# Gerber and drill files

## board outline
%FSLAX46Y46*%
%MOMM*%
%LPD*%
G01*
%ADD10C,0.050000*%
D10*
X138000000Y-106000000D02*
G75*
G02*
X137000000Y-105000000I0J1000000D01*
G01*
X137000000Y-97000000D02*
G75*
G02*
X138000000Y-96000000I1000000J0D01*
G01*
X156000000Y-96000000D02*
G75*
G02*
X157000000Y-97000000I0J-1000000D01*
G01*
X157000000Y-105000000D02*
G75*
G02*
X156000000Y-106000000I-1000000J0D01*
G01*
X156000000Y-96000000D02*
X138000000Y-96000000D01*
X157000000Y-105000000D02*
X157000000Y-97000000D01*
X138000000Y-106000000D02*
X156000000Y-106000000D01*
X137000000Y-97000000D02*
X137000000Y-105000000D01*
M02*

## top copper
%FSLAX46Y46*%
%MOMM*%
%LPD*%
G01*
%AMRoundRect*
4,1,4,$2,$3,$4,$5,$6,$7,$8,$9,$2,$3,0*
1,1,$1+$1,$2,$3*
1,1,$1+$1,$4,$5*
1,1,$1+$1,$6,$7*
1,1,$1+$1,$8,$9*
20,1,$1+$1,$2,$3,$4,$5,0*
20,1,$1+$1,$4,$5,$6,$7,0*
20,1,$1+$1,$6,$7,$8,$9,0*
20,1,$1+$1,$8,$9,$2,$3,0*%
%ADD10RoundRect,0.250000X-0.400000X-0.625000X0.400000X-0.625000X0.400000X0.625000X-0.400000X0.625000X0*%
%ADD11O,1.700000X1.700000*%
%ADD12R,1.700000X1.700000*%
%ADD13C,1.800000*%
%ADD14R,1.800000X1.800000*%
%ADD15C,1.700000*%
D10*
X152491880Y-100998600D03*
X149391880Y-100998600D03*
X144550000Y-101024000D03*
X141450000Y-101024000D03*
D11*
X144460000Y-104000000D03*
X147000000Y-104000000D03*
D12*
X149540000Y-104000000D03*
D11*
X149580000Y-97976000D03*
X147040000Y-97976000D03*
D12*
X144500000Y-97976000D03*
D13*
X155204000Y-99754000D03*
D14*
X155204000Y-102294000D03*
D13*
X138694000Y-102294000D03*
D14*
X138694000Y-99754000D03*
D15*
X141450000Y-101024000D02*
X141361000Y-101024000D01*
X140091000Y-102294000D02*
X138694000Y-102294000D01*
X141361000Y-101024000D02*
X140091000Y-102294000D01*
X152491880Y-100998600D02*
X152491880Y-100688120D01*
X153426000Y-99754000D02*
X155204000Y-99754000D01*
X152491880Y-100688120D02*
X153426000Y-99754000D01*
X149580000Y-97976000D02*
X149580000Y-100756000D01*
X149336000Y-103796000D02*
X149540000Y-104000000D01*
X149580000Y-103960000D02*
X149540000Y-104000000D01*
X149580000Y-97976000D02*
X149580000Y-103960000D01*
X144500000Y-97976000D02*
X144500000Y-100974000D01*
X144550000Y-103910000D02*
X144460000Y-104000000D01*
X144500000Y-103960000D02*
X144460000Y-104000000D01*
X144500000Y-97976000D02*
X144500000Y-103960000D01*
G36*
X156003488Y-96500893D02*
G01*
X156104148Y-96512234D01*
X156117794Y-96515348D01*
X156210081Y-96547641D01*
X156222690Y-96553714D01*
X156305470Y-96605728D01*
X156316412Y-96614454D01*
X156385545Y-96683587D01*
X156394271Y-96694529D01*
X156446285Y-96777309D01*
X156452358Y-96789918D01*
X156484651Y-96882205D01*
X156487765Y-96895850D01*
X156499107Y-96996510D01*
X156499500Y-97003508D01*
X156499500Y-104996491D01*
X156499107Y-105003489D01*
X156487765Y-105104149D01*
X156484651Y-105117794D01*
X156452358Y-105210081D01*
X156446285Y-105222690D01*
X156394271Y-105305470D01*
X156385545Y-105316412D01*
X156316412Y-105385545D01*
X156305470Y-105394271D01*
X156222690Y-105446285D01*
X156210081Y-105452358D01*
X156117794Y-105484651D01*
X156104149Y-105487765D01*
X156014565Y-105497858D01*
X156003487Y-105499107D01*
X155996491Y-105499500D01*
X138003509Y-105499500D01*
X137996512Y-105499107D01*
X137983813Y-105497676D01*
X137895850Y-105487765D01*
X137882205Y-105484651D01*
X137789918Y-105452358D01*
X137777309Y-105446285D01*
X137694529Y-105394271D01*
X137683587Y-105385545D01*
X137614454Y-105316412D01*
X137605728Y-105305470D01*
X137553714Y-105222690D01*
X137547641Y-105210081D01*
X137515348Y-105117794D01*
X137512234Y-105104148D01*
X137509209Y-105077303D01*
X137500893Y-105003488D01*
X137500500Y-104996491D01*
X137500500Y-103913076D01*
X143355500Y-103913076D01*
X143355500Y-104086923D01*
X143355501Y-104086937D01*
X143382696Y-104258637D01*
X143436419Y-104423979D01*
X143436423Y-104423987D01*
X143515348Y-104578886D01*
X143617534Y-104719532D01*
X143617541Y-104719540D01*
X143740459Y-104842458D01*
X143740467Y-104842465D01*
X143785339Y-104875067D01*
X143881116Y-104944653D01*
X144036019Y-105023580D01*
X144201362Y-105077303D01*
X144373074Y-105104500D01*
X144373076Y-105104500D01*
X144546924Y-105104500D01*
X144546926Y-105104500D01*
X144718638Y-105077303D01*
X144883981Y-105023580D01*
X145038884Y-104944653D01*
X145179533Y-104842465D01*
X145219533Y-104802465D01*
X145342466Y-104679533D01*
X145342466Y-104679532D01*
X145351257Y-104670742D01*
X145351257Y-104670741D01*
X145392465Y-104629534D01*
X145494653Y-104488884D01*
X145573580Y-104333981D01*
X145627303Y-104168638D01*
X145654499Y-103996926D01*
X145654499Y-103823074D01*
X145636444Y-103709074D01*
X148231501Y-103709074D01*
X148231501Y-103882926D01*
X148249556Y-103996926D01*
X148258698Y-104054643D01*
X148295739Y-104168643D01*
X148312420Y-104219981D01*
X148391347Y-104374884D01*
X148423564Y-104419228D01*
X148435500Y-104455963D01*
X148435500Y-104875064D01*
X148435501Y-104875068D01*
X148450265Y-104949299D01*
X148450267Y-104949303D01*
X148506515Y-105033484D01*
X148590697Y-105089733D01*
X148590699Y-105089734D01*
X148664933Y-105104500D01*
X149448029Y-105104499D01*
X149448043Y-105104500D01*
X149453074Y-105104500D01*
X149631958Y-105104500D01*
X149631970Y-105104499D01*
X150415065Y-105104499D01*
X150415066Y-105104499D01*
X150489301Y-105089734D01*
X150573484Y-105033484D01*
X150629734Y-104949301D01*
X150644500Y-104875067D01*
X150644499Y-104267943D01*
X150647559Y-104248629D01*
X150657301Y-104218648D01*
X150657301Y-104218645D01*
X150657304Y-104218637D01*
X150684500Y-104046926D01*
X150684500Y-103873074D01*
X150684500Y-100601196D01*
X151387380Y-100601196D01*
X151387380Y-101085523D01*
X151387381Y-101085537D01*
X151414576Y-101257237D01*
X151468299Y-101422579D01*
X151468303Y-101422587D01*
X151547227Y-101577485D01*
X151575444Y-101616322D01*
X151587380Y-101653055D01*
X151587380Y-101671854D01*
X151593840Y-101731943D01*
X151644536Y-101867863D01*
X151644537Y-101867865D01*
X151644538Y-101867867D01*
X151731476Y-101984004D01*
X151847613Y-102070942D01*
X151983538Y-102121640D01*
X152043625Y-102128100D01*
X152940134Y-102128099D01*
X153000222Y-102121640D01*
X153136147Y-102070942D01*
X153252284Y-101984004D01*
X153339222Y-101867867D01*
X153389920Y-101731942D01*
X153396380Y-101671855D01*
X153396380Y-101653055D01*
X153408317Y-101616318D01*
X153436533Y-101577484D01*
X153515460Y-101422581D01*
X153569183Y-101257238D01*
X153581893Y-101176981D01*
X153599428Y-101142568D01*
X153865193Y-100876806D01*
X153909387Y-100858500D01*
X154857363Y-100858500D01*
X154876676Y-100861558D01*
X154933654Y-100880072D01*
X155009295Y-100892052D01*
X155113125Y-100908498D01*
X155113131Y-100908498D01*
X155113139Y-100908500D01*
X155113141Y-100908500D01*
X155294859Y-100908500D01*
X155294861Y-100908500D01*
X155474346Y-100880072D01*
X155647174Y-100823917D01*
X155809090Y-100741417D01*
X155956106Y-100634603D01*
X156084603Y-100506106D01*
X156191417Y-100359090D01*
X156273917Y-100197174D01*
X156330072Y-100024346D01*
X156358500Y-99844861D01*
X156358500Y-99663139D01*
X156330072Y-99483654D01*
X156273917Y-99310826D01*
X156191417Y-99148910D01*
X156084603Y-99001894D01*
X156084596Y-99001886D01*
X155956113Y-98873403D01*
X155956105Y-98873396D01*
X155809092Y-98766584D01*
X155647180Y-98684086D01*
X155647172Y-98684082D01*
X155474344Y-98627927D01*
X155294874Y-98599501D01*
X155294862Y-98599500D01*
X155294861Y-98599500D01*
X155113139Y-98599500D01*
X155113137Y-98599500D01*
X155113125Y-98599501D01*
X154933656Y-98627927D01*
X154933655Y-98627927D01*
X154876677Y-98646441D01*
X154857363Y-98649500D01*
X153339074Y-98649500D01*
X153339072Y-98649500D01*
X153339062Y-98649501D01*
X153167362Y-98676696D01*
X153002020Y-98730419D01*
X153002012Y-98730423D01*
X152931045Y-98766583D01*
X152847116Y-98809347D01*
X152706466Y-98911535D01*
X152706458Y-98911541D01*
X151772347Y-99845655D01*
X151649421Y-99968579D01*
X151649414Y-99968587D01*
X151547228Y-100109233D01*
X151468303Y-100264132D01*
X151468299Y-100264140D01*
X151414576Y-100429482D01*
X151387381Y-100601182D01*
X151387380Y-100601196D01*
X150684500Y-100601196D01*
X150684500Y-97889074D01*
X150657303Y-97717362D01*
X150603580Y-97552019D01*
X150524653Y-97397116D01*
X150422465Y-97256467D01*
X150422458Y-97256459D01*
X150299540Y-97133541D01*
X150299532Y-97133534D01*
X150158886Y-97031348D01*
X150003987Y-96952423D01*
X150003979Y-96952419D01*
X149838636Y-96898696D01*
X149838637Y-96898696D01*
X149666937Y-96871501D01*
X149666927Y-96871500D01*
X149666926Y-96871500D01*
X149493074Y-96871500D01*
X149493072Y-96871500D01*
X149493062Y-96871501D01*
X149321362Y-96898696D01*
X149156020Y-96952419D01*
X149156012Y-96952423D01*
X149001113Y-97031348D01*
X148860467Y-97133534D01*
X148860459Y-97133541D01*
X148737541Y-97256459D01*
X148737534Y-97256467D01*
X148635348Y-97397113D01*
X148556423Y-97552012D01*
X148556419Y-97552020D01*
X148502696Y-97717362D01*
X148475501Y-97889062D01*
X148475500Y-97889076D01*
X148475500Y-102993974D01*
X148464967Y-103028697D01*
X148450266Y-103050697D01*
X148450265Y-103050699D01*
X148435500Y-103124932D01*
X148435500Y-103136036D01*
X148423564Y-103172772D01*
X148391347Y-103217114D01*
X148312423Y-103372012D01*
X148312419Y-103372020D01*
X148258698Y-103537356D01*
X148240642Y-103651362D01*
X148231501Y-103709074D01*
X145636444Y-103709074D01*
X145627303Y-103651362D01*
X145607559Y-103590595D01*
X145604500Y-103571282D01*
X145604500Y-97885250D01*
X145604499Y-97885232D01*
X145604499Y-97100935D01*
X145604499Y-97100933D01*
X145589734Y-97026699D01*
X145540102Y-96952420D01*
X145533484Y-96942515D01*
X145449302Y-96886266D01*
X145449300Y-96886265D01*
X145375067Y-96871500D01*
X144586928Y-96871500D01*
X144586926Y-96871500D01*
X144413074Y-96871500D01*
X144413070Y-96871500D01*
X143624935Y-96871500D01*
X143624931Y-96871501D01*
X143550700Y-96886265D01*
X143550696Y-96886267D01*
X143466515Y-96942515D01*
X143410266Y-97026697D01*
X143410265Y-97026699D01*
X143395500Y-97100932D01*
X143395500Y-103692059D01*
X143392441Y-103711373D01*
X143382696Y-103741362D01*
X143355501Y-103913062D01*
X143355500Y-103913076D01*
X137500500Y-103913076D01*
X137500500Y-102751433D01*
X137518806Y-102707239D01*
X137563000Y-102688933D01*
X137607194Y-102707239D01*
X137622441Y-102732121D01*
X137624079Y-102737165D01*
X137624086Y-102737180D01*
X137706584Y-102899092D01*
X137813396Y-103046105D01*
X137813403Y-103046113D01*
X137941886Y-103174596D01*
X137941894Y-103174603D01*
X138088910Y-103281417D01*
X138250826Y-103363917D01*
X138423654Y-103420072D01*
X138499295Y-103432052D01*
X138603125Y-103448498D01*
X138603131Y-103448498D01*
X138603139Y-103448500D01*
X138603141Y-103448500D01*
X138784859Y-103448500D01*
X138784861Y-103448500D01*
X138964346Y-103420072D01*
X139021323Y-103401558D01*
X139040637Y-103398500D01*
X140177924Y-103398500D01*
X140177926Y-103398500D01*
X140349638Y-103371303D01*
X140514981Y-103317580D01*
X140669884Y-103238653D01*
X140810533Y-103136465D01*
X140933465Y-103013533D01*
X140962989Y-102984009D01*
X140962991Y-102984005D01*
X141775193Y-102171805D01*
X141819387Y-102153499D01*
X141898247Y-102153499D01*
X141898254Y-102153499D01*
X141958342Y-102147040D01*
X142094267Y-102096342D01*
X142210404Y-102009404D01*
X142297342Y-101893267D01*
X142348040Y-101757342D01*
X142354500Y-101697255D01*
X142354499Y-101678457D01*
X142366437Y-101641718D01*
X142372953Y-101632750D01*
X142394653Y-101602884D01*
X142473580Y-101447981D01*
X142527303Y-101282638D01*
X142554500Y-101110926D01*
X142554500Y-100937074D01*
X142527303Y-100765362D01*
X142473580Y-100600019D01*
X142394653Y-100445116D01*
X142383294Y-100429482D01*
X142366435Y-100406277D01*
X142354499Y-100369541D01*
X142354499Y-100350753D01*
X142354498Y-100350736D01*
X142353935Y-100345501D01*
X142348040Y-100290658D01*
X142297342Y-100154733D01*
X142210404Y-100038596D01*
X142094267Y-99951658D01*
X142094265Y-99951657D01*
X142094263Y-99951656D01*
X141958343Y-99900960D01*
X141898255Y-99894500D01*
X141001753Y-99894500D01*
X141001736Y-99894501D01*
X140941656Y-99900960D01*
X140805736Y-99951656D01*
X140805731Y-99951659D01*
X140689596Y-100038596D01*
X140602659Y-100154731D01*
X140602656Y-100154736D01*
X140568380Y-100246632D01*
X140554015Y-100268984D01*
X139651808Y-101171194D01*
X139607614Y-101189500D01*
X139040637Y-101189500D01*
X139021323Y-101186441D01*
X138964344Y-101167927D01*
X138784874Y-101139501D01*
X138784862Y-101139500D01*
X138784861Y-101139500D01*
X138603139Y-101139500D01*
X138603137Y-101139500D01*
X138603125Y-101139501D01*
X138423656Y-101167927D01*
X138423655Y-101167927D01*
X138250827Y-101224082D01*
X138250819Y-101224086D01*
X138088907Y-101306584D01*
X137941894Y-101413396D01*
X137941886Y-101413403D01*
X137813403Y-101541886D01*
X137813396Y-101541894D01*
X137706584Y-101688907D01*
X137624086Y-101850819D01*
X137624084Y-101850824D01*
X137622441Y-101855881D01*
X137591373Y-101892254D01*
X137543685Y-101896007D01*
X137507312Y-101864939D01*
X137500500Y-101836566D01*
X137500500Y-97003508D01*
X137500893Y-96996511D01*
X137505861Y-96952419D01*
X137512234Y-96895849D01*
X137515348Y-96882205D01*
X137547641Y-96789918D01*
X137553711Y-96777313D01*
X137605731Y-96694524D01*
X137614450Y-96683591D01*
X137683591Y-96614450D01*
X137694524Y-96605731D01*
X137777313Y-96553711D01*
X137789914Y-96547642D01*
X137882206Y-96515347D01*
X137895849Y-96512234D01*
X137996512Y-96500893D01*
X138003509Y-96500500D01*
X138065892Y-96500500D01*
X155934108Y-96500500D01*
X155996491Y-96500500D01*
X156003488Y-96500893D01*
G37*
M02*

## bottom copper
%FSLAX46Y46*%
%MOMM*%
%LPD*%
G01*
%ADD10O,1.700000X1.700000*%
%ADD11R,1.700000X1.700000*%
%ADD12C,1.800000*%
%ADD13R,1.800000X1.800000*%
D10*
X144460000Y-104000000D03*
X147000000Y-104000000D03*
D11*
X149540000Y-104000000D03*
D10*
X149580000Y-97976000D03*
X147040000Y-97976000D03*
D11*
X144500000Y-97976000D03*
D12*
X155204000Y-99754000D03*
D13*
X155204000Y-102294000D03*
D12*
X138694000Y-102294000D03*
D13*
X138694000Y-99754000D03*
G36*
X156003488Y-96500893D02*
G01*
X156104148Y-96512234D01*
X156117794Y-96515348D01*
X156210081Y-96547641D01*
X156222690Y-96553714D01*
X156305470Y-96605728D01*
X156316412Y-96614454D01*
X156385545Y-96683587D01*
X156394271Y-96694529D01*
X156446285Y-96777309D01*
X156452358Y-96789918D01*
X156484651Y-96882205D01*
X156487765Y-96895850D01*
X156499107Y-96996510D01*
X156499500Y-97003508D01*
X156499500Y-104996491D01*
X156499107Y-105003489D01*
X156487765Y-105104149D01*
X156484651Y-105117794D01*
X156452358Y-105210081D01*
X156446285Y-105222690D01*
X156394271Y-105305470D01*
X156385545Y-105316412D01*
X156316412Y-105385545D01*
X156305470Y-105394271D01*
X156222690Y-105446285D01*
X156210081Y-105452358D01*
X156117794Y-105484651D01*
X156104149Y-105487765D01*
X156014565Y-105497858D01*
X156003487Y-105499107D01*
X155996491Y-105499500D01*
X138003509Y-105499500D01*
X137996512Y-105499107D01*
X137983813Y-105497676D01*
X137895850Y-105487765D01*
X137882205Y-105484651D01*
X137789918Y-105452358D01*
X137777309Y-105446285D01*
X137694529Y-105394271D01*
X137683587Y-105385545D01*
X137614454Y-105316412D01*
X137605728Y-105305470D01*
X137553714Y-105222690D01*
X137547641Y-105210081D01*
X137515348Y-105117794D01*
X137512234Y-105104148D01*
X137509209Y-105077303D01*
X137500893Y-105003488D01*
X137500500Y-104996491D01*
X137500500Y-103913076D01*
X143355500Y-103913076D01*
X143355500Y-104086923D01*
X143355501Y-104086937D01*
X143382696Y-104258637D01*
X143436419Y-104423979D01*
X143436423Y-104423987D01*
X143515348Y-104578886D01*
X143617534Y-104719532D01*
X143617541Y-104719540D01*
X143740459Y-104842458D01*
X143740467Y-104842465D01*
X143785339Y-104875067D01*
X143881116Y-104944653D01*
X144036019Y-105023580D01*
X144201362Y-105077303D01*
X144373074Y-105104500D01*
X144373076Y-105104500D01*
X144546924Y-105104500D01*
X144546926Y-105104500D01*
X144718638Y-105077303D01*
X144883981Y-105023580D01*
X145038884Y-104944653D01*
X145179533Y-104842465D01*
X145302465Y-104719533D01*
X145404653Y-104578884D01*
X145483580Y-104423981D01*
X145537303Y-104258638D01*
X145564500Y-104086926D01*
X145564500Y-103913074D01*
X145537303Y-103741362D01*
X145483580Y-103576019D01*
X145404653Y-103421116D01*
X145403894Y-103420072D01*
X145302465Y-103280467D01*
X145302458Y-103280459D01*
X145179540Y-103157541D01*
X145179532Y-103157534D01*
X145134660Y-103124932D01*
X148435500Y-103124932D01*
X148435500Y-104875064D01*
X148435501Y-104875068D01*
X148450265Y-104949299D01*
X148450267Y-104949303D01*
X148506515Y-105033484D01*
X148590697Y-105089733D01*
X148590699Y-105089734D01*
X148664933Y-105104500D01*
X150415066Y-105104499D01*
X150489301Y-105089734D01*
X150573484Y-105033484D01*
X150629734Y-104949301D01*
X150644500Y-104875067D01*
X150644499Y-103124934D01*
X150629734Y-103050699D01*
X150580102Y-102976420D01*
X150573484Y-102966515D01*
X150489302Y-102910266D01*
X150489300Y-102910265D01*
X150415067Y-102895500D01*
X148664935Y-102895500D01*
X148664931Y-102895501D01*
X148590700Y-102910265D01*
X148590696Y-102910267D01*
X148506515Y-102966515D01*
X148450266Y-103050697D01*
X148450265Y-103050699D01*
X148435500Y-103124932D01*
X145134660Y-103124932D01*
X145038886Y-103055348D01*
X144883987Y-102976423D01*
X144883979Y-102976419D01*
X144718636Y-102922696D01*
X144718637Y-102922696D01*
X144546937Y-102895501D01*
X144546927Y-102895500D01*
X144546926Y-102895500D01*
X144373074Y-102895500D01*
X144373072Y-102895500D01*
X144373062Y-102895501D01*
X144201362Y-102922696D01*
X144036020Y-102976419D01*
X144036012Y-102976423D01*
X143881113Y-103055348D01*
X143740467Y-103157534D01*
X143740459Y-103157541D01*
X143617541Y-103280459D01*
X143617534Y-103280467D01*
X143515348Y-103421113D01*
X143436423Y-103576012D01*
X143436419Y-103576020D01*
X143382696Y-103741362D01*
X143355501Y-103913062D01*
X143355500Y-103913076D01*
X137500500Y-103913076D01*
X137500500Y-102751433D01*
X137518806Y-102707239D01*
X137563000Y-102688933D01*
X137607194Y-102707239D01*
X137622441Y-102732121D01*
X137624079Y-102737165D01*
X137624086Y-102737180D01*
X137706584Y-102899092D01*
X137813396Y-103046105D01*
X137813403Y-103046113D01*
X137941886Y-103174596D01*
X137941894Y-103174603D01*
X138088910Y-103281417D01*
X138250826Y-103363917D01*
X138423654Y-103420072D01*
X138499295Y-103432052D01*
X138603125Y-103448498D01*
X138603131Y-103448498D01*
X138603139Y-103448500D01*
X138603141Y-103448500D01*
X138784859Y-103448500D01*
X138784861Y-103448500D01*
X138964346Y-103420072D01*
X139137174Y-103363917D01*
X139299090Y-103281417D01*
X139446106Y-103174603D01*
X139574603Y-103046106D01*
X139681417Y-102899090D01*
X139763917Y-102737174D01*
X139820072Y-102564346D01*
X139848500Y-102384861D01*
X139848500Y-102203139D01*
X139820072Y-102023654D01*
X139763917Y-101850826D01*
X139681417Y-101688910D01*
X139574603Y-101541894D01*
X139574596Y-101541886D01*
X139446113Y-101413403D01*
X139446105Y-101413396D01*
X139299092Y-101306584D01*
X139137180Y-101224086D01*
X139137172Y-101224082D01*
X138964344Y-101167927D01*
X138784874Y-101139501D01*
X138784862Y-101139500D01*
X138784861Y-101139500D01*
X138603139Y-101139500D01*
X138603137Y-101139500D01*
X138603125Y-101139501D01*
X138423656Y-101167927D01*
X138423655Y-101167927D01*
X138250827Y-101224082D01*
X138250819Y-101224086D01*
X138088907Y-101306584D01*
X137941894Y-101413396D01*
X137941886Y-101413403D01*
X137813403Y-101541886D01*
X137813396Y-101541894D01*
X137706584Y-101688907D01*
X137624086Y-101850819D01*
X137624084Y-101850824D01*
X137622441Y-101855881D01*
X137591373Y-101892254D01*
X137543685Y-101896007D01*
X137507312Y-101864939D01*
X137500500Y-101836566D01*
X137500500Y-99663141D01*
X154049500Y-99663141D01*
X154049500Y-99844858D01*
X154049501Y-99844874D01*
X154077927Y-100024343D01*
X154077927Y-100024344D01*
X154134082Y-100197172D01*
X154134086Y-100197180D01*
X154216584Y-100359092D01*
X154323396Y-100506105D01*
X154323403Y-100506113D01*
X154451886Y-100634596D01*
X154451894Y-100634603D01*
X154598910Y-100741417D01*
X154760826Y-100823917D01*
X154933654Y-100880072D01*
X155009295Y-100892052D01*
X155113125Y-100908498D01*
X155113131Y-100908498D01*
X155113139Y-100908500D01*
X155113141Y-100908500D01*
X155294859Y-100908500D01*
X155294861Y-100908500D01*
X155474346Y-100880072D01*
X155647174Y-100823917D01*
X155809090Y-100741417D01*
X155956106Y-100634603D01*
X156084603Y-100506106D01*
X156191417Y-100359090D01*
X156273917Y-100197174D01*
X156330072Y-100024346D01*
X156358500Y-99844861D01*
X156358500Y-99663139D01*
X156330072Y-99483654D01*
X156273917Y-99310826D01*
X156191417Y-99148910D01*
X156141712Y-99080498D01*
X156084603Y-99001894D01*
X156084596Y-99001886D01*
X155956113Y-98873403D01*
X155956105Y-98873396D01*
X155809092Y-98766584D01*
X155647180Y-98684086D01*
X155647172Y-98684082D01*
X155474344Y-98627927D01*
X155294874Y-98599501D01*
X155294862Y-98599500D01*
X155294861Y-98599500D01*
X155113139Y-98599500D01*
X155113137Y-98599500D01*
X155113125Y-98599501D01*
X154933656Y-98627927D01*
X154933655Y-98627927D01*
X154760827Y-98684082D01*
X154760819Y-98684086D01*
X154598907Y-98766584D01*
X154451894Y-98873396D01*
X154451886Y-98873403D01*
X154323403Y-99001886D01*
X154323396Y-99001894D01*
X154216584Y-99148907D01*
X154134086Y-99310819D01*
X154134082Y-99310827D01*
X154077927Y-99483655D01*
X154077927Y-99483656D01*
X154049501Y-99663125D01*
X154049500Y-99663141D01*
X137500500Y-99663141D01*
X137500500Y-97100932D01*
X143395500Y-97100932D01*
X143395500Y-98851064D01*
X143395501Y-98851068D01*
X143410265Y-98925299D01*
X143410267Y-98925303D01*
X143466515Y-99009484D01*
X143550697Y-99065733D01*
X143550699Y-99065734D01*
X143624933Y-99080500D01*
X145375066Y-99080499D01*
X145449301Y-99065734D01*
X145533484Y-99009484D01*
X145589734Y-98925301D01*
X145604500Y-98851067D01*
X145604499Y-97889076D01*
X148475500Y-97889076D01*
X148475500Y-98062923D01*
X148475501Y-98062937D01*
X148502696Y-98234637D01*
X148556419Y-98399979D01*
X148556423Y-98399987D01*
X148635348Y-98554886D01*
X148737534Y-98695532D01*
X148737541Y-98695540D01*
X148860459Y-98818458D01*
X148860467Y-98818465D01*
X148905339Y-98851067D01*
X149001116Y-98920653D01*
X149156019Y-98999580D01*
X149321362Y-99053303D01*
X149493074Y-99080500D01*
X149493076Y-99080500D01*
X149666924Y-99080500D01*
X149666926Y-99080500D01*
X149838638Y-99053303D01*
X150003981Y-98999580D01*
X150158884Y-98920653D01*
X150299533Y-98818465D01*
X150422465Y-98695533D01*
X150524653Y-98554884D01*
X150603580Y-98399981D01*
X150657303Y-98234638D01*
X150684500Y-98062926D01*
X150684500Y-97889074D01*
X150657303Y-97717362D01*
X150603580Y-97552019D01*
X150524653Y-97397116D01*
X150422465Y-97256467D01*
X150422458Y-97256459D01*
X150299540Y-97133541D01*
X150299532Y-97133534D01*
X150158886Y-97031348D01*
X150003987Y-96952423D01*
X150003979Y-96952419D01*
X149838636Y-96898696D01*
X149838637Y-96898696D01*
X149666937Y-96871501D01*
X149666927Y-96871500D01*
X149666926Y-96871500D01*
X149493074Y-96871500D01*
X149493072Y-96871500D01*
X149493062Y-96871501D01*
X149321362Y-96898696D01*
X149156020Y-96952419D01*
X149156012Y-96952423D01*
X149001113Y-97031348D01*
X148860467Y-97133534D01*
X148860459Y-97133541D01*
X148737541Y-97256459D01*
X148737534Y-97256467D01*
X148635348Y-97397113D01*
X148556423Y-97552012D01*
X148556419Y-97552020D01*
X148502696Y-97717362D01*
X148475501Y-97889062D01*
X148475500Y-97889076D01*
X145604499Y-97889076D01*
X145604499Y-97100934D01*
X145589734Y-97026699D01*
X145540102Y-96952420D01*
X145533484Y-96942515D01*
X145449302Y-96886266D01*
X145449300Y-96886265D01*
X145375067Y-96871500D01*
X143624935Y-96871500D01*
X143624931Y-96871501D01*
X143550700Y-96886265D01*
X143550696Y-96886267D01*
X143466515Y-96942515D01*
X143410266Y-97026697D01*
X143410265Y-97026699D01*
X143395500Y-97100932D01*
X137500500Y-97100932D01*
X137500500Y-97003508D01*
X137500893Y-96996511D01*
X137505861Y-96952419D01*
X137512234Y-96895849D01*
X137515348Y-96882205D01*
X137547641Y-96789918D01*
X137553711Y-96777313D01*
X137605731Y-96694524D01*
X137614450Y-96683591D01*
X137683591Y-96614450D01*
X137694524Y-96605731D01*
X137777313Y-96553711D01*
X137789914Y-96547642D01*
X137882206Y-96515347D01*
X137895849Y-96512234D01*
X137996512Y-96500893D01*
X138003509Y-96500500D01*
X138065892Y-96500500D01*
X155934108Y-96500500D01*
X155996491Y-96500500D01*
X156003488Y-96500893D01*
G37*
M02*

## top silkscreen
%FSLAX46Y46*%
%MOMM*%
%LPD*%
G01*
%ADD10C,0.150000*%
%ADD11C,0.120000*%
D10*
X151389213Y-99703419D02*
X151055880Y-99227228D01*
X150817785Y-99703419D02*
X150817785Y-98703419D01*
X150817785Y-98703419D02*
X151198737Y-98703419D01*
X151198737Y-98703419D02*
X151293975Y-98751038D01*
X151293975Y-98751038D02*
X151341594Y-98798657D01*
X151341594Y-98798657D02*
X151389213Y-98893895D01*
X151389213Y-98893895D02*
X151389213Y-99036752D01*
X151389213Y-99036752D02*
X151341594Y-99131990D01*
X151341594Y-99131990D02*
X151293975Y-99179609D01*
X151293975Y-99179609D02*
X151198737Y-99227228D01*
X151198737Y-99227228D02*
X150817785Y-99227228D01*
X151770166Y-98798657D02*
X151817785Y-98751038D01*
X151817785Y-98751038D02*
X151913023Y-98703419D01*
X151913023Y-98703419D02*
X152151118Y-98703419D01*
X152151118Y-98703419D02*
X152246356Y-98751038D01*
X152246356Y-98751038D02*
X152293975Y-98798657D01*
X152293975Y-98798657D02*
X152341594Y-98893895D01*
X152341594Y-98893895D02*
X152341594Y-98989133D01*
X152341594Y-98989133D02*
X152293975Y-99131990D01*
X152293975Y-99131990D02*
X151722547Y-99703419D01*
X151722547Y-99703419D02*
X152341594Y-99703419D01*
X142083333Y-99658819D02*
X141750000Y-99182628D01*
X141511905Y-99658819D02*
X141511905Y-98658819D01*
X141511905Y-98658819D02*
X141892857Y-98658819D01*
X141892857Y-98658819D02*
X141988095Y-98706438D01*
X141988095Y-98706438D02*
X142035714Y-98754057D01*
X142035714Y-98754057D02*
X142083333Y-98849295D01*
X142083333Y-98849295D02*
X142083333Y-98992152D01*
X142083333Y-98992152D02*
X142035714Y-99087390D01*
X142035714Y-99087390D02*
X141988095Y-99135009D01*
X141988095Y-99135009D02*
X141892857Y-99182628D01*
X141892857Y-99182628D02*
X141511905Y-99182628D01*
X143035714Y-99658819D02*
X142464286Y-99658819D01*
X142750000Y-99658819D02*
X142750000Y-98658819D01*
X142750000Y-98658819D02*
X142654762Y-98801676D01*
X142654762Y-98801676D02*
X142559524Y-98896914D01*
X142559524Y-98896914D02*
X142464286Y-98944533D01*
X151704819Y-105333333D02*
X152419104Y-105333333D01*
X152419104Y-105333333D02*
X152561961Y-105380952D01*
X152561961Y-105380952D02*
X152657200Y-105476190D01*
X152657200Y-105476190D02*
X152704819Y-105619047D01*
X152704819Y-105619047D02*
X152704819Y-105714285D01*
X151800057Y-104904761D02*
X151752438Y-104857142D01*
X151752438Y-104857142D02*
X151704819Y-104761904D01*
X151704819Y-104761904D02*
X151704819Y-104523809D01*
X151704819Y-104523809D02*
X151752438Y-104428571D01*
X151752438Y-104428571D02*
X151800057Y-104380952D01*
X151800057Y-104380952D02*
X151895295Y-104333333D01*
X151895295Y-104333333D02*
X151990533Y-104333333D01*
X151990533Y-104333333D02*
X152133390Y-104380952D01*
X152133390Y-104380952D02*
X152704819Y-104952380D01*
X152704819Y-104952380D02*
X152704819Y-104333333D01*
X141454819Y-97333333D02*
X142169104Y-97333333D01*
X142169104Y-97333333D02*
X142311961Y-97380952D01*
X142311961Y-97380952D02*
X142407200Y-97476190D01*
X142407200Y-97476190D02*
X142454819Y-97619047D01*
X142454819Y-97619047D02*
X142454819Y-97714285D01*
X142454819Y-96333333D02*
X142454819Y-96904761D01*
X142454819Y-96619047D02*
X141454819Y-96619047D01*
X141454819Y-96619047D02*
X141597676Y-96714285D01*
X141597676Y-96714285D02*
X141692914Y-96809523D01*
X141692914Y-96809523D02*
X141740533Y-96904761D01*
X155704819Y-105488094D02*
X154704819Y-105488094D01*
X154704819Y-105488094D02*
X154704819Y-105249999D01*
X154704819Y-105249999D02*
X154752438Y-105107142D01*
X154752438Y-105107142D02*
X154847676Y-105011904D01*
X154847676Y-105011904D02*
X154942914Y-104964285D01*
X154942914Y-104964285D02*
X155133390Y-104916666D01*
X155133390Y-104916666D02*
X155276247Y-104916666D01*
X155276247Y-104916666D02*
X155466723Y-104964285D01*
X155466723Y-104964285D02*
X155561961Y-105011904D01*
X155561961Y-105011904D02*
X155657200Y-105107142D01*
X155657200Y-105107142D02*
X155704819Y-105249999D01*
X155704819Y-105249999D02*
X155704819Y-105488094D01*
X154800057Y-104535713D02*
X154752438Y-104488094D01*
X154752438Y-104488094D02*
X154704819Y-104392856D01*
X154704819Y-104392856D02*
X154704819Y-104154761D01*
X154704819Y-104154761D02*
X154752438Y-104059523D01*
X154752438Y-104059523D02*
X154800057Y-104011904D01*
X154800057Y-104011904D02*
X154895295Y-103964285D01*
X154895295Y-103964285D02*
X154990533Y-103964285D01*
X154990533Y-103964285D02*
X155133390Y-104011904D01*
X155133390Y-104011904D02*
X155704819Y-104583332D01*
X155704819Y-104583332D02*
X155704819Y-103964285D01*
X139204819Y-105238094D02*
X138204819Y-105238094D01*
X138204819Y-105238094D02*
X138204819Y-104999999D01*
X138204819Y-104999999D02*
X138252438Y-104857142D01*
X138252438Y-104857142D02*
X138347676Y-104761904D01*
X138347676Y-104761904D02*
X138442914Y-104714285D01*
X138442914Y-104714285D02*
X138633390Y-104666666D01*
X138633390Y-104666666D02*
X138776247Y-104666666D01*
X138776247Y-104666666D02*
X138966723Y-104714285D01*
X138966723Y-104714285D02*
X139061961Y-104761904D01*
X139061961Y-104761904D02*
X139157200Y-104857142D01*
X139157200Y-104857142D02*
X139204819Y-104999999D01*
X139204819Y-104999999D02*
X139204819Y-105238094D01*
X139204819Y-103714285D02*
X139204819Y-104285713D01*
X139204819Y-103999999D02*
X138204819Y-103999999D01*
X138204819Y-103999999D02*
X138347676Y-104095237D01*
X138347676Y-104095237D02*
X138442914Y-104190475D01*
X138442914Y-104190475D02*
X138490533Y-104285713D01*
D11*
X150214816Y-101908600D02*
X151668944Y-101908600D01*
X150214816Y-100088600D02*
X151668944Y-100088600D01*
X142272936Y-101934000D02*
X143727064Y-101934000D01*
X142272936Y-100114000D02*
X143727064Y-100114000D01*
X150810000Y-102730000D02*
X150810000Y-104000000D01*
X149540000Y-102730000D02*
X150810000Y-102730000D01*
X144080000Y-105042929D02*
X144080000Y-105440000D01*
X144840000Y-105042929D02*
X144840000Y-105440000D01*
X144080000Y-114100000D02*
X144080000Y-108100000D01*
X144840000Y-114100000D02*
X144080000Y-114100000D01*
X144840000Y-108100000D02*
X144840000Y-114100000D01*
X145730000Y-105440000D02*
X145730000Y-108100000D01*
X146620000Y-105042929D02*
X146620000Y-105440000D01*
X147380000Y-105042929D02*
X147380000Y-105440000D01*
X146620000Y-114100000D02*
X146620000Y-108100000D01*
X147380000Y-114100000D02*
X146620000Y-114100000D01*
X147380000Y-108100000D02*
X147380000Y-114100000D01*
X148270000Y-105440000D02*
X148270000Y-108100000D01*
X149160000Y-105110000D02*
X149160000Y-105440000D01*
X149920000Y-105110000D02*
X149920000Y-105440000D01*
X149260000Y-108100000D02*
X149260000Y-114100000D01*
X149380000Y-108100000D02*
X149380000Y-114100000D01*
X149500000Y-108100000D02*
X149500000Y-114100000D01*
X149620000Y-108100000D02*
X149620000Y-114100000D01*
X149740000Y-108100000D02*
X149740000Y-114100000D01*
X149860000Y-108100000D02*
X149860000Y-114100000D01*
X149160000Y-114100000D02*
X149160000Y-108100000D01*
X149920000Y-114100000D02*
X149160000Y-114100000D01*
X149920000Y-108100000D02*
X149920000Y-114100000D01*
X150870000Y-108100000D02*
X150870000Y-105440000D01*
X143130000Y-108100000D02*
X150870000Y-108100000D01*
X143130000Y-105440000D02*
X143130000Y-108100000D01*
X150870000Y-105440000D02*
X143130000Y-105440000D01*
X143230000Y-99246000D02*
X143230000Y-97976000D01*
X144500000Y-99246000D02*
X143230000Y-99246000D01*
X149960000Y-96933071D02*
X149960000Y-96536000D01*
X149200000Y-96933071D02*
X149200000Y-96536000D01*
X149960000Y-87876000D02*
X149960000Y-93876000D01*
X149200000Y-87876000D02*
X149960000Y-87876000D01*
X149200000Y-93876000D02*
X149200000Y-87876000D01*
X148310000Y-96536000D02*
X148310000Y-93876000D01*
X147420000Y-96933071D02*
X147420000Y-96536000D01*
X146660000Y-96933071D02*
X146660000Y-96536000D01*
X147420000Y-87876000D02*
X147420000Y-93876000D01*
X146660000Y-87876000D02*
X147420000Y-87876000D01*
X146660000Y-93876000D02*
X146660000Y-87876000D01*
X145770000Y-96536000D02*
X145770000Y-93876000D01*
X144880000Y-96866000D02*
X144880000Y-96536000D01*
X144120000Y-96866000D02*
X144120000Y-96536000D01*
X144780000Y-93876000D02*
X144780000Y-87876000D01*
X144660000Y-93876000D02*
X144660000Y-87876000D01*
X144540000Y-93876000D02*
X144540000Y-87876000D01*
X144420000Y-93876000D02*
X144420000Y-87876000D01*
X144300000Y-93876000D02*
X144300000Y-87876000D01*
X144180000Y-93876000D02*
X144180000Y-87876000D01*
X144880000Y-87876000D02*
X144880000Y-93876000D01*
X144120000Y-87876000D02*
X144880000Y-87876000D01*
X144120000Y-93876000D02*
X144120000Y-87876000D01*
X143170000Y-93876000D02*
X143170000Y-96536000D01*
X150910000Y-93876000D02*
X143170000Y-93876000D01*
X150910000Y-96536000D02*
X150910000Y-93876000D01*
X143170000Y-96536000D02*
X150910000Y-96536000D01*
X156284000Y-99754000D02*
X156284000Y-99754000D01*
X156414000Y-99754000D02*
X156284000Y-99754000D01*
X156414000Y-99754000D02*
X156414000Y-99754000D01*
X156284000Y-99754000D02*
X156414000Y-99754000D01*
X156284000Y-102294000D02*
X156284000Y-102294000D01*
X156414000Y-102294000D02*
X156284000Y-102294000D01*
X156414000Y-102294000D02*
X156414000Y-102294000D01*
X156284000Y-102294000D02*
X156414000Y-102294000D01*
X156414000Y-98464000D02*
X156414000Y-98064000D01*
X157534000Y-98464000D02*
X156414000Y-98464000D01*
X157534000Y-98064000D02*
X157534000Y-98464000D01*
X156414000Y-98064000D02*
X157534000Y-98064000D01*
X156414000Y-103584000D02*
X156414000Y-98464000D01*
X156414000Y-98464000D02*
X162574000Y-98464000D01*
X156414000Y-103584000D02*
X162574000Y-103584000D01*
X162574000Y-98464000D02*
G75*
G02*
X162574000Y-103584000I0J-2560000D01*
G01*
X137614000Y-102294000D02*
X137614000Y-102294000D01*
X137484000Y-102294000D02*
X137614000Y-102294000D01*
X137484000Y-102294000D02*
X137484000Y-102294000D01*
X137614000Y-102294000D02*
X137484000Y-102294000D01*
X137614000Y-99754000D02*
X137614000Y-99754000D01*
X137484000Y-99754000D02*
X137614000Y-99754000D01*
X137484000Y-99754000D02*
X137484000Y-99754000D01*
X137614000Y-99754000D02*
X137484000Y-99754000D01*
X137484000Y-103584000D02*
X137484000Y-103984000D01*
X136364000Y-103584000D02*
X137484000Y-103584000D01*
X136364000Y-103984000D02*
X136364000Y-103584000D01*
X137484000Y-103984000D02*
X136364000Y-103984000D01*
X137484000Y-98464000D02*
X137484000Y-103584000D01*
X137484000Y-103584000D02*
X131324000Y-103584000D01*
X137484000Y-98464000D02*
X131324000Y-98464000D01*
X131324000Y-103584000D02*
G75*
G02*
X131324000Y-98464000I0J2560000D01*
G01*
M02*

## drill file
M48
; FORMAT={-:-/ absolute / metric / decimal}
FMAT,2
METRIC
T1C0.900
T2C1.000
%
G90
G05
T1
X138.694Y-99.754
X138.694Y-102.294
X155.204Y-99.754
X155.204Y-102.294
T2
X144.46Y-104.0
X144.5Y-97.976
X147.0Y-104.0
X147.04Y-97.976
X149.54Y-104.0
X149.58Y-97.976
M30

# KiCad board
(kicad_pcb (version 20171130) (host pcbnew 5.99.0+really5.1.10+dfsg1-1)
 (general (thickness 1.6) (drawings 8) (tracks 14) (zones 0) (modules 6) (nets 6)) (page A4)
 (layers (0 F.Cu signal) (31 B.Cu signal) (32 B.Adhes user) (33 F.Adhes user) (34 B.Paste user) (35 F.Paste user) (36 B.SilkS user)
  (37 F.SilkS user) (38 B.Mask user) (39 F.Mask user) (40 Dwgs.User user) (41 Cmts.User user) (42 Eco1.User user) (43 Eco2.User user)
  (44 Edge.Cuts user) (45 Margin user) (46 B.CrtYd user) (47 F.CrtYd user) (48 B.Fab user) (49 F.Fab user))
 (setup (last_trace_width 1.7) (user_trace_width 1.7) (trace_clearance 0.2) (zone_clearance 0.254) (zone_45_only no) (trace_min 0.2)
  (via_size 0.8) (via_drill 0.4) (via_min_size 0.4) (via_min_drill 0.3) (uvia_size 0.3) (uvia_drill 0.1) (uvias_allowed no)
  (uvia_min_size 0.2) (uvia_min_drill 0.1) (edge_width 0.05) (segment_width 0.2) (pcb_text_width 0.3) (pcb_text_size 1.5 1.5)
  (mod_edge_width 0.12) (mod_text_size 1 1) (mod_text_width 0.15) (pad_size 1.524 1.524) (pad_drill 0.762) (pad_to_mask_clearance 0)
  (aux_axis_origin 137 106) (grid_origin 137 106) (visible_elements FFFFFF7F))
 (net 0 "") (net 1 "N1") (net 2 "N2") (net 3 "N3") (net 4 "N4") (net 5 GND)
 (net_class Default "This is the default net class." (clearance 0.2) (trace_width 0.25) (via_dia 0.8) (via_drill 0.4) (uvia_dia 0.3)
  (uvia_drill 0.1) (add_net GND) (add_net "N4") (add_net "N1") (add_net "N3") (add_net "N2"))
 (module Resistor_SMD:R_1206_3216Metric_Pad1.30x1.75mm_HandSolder (layer F.Cu) (at 150.94188 100.9986)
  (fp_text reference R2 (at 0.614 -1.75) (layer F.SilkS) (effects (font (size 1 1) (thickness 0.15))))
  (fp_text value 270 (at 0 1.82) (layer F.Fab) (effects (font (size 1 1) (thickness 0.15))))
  (fp_line (start -0.727064 0.91) (end 0.727064 0.91) (layer F.SilkS) (width 0.12))
  (fp_line (start -0.727064 -0.91) (end 0.727064 -0.91) (layer F.SilkS) (width 0.12))
  (pad 2 smd roundrect (at 1.55 0) (size 1.3 1.75) (layers F.Cu F.Paste F.Mask) (roundrect_rratio 0.192308) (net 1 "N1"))
  (pad 1 smd roundrect (at -1.55 0) (size 1.3 1.75) (layers F.Cu F.Paste F.Mask) (roundrect_rratio 0.192308) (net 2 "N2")))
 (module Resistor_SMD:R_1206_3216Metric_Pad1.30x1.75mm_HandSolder (layer F.Cu) (at 143 101.024)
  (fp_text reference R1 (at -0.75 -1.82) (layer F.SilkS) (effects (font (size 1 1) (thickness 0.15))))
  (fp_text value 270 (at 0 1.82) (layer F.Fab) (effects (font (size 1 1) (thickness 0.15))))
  (fp_line (start -0.727064 0.91) (end 0.727064 0.91) (layer F.SilkS) (width 0.12))
  (fp_line (start -0.727064 -0.91) (end 0.727064 -0.91) (layer F.SilkS) (width 0.12))
  (pad 2 smd roundrect (at 1.55 0) (size 1.3 1.75) (layers F.Cu F.Paste F.Mask) (roundrect_rratio 0.192308) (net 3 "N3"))
  (pad 1 smd roundrect (at -1.55 0) (size 1.3 1.75) (layers F.Cu F.Paste F.Mask) (roundrect_rratio 0.192308) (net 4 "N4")))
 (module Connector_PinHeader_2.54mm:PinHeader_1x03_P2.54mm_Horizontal (layer F.Cu) (at 149.54 104 270)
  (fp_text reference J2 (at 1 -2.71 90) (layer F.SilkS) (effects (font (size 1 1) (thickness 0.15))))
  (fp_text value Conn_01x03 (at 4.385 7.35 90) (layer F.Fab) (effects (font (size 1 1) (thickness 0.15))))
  (fp_line (start -1.27 -1.27) (end 0 -1.27) (layer F.SilkS) (width 0.12))
  (fp_line (start -1.27 0) (end -1.27 -1.27) (layer F.SilkS) (width 0.12))
  (fp_line (start 1.042929 5.46) (end 1.44 5.46) (layer F.SilkS) (width 0.12))
  (fp_line (start 1.042929 4.7) (end 1.44 4.7) (layer F.SilkS) (width 0.12))
  (fp_line (start 10.1 5.46) (end 4.1 5.46) (layer F.SilkS) (width 0.12))
  (fp_line (start 10.1 4.7) (end 10.1 5.46) (layer F.SilkS) (width 0.12))
  (fp_line (start 4.1 4.7) (end 10.1 4.7) (layer F.SilkS) (width 0.12))
  (fp_line (start 1.44 3.81) (end 4.1 3.81) (layer F.SilkS) (width 0.12))
  (fp_line (start 1.042929 2.92) (end 1.44 2.92) (layer F.SilkS) (width 0.12))
  (fp_line (start 1.042929 2.16) (end 1.44 2.16) (layer F.SilkS) (width 0.12))
  (fp_line (start 10.1 2.92) (end 4.1 2.92) (layer F.SilkS) (width 0.12))
  (fp_line (start 10.1 2.16) (end 10.1 2.92) (layer F.SilkS) (width 0.12))
  (fp_line (start 4.1 2.16) (end 10.1 2.16) (layer F.SilkS) (width 0.12))
  (fp_line (start 1.44 1.27) (end 4.1 1.27) (layer F.SilkS) (width 0.12))
  (fp_line (start 1.11 0.38) (end 1.44 0.38) (layer F.SilkS) (width 0.12))
  (fp_line (start 1.11 -0.38) (end 1.44 -0.38) (layer F.SilkS) (width 0.12))
  (fp_line (start 4.1 0.28) (end 10.1 0.28) (layer F.SilkS) (width 0.12))
  (fp_line (start 4.1 0.16) (end 10.1 0.16) (layer F.SilkS) (width 0.12))
  (fp_line (start 4.1 0.04) (end 10.1 0.04) (layer F.SilkS) (width 0.12))
  (fp_line (start 4.1 -0.08) (end 10.1 -0.08) (layer F.SilkS) (width 0.12))
  (fp_line (start 4.1 -0.2) (end 10.1 -0.2) (layer F.SilkS) (width 0.12))
  (fp_line (start 4.1 -0.32) (end 10.1 -0.32) (layer F.SilkS) (width 0.12))
  (fp_line (start 10.1 0.38) (end 4.1 0.38) (layer F.SilkS) (width 0.12))
  (fp_line (start 10.1 -0.38) (end 10.1 0.38) (layer F.SilkS) (width 0.12))
  (fp_line (start 4.1 -0.38) (end 10.1 -0.38) (layer F.SilkS) (width 0.12))
  (fp_line (start 4.1 -1.33) (end 1.44 -1.33) (layer F.SilkS) (width 0.12))
  (fp_line (start 4.1 6.41) (end 4.1 -1.33) (layer F.SilkS) (width 0.12))
  (fp_line (start 1.44 6.41) (end 4.1 6.41) (layer F.SilkS) (width 0.12))
  (fp_line (start 1.44 -1.33) (end 1.44 6.41) (layer F.SilkS) (width 0.12))
  (pad 3 thru_hole oval (at 0 5.08 270) (size 1.7 1.7) (drill 1) (layers *.Cu *.Mask) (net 3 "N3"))
  (pad 2 thru_hole oval (at 0 2.54 270) (size 1.7 1.7) (drill 1) (layers *.Cu *.Mask) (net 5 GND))
  (pad 1 thru_hole rect (at 0 0 270) (size 1.7 1.7) (drill 1) (layers *.Cu *.Mask) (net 2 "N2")))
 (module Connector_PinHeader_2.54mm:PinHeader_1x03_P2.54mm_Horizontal (layer F.Cu) (at 144.5 97.976 90)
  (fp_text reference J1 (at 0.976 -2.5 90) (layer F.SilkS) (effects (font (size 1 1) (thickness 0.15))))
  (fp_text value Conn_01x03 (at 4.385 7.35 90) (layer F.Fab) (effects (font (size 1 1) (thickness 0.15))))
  (fp_line (start -1.27 -1.27) (end 0 -1.27) (layer F.SilkS) (width 0.12))
  (fp_line (start -1.27 0) (end -1.27 -1.27) (layer F.SilkS) (width 0.12))
  (fp_line (start 1.042929 5.46) (end 1.44 5.46) (layer F.SilkS) (width 0.12))
  (fp_line (start 1.042929 4.7) (end 1.44 4.7) (layer F.SilkS) (width 0.12))
  (fp_line (start 10.1 5.46) (end 4.1 5.46) (layer F.SilkS) (width 0.12))
  (fp_line (start 10.1 4.7) (end 10.1 5.46) (layer F.SilkS) (width 0.12))
  (fp_line (start 4.1 4.7) (end 10.1 4.7) (layer F.SilkS) (width 0.12))
  (fp_line (start 1.44 3.81) (end 4.1 3.81) (layer F.SilkS) (width 0.12))
  (fp_line (start 1.042929 2.92) (end 1.44 2.92) (layer F.SilkS) (width 0.12))
  (fp_line (start 1.042929 2.16) (end 1.44 2.16) (layer F.SilkS) (width 0.12))
  (fp_line (start 10.1 2.92) (end 4.1 2.92) (layer F.SilkS) (width 0.12))
  (fp_line (start 10.1 2.16) (end 10.1 2.92) (layer F.SilkS) (width 0.12))
  (fp_line (start 4.1 2.16) (end 10.1 2.16) (layer F.SilkS) (width 0.12))
  (fp_line (start 1.44 1.27) (end 4.1 1.27) (layer F.SilkS) (width 0.12))
  (fp_line (start 1.11 0.38) (end 1.44 0.38) (layer F.SilkS) (width 0.12))
  (fp_line (start 1.11 -0.38) (end 1.44 -0.38) (layer F.SilkS) (width 0.12))
  (fp_line (start 4.1 0.28) (end 10.1 0.28) (layer F.SilkS) (width 0.12))
  (fp_line (start 4.1 0.16) (end 10.1 0.16) (layer F.SilkS) (width 0.12))
  (fp_line (start 4.1 0.04) (end 10.1 0.04) (layer F.SilkS) (width 0.12))
  (fp_line (start 4.1 -0.08) (end 10.1 -0.08) (layer F.SilkS) (width 0.12))
  (fp_line (start 4.1 -0.2) (end 10.1 -0.2) (layer F.SilkS) (width 0.12))
  (fp_line (start 4.1 -0.32) (end 10.1 -0.32) (layer F.SilkS) (width 0.12))
  (fp_line (start 10.1 0.38) (end 4.1 0.38) (layer F.SilkS) (width 0.12))
  (fp_line (start 10.1 -0.38) (end 10.1 0.38) (layer F.SilkS) (width 0.12))
  (fp_line (start 4.1 -0.38) (end 10.1 -0.38) (layer F.SilkS) (width 0.12))
  (fp_line (start 4.1 -1.33) (end 1.44 -1.33) (layer F.SilkS) (width 0.12))
  (fp_line (start 4.1 6.41) (end 4.1 -1.33) (layer F.SilkS) (width 0.12))
  (fp_line (start 1.44 6.41) (end 4.1 6.41) (layer F.SilkS) (width 0.12))
  (fp_line (start 1.44 -1.33) (end 1.44 6.41) (layer F.SilkS) (width 0.12))
  (pad 3 thru_hole oval (at 0 5.08 90) (size 1.7 1.7) (drill 1) (layers *.Cu *.Mask) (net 2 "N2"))
  (pad 2 thru_hole oval (at 0 2.54 90) (size 1.7 1.7) (drill 1) (layers *.Cu *.Mask) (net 5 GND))
  (pad 1 thru_hole rect (at 0 0 90) (size 1.7 1.7) (drill 1) (layers *.Cu *.Mask) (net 3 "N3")))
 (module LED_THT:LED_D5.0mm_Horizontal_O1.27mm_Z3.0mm (layer F.Cu) (at 155.204 102.294 90)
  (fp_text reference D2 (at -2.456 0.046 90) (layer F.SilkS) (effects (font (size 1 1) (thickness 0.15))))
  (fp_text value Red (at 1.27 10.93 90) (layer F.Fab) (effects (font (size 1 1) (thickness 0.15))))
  (fp_line (start 2.54 1.08) (end 2.54 1.08) (layer F.SilkS) (width 0.12))
  (fp_line (start 2.54 1.21) (end 2.54 1.08) (layer F.SilkS) (width 0.12))
  (fp_line (start 2.54 1.21) (end 2.54 1.21) (layer F.SilkS) (width 0.12))
  (fp_line (start 2.54 1.08) (end 2.54 1.21) (layer F.SilkS) (width 0.12))
  (fp_line (start 0 1.08) (end 0 1.08) (layer F.SilkS) (width 0.12))
  (fp_line (start 0 1.21) (end 0 1.08) (layer F.SilkS) (width 0.12))
  (fp_line (start 0 1.21) (end 0 1.21) (layer F.SilkS) (width 0.12))
  (fp_line (start 0 1.08) (end 0 1.21) (layer F.SilkS) (width 0.12))
  (fp_line (start 3.83 1.21) (end 4.23 1.21) (layer F.SilkS) (width 0.12))
  (fp_line (start 3.83 2.33) (end 3.83 1.21) (layer F.SilkS) (width 0.12))
  (fp_line (start 4.23 2.33) (end 3.83 2.33) (layer F.SilkS) (width 0.12))
  (fp_line (start 4.23 1.21) (end 4.23 2.33) (layer F.SilkS) (width 0.12))
  (fp_line (start -1.29 1.21) (end 3.83 1.21) (layer F.SilkS) (width 0.12))
  (fp_line (start 3.83 1.21) (end 3.83 7.37) (layer F.SilkS) (width 0.12))
  (fp_line (start -1.29 1.21) (end -1.29 7.37) (layer F.SilkS) (width 0.12))
  (fp_arc (start 1.27 7.37) (end -1.29 7.37) (angle -180) (layer F.SilkS) (width 0.12))
  (pad 2 thru_hole circle (at 2.54 0 90) (size 1.8 1.8) (drill 0.9) (layers *.Cu *.Mask) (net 1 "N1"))
  (pad 1 thru_hole rect (at 0 0 90) (size 1.8 1.8) (drill 0.9) (layers *.Cu *.Mask) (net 5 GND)))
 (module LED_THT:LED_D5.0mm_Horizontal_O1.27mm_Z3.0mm (layer F.Cu) (at 138.694 99.754 270)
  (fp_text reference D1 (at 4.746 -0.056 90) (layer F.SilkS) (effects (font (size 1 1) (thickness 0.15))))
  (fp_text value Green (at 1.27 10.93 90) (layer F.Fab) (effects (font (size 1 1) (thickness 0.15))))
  (fp_line (start 2.54 1.08) (end 2.54 1.08) (layer F.SilkS) (width 0.12))
  (fp_line (start 2.54 1.21) (end 2.54 1.08) (layer F.SilkS) (width 0.12))
  (fp_line (start 2.54 1.21) (end 2.54 1.21) (layer F.SilkS) (width 0.12))
  (fp_line (start 2.54 1.08) (end 2.54 1.21) (layer F.SilkS) (width 0.12))
  (fp_line (start 0 1.08) (end 0 1.08) (layer F.SilkS) (width 0.12))
  (fp_line (start 0 1.21) (end 0 1.08) (layer F.SilkS) (width 0.12))
  (fp_line (start 0 1.21) (end 0 1.21) (layer F.SilkS) (width 0.12))
  (fp_line (start 0 1.08) (end 0 1.21) (layer F.SilkS) (width 0.12))
  (fp_line (start 3.83 1.21) (end 4.23 1.21) (layer F.SilkS) (width 0.12))
  (fp_line (start 3.83 2.33) (end 3.83 1.21) (layer F.SilkS) (width 0.12))
  (fp_line (start 4.23 2.33) (end 3.83 2.33) (layer F.SilkS) (width 0.12))
  (fp_line (start 4.23 1.21) (end 4.23 2.33) (layer F.SilkS) (width 0.12))
  (fp_line (start -1.29 1.21) (end 3.83 1.21) (layer F.SilkS) (width 0.12))
  (fp_line (start 3.83 1.21) (end 3.83 7.37) (layer F.SilkS) (width 0.12))
  (fp_line (start -1.29 1.21) (end -1.29 7.37) (layer F.SilkS) (width 0.12))
  (fp_arc (start 1.27 7.37) (end -1.29 7.37) (angle -180) (layer F.SilkS) (width 0.12))
  (pad 2 thru_hole circle (at 2.54 0 270) (size 1.8 1.8) (drill 0.9) (layers *.Cu *.Mask) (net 4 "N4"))
  (pad 1 thru_hole rect (at 0 0 270) (size 1.8 1.8) (drill 0.9) (layers *.Cu *.Mask) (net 5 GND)))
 (gr_arc (start 138 105) (end 137 105) (angle -90) (layer Edge.Cuts) (width 0.05))
 (gr_arc (start 138 97) (end 138 96) (angle -90) (layer Edge.Cuts) (width 0.05))
 (gr_arc (start 156 97) (end 157 97) (angle -90) (layer Edge.Cuts) (width 0.05))
 (gr_arc (start 156 105) (end 156 106) (angle -90) (layer Edge.Cuts) (width 0.05))
 (gr_line (start 156 96) (end 138 96) (layer Edge.Cuts) (width 0.05))
 (gr_line (start 157 105) (end 157 97) (layer Edge.Cuts) (width 0.05))
 (gr_line (start 138 106) (end 156 106) (layer Edge.Cuts) (width 0.05))
 (gr_line (start 137 97) (end 137 105) (layer Edge.Cuts) (width 0.05))
 (segment (start 141.45 101.024) (end 141.361 101.024) (width 1.7) (layer F.Cu) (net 4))
 (segment (start 140.091 102.294) (end 138.694 102.294) (width 1.7) (layer F.Cu) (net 4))
 (segment (start 141.361 101.024) (end 140.091 102.294) (width 1.7) (layer F.Cu) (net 4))
 (segment (start 152.49188 100.9986) (end 152.49188 100.68812) (width 1.7) (layer F.Cu) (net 1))
 (segment (start 153.426 99.754) (end 155.204 99.754) (width 1.7) (layer F.Cu) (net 1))
 (segment (start 152.49188 100.68812) (end 153.426 99.754) (width 1.7) (layer F.Cu) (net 1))
 (segment (start 149.58 97.976) (end 149.58 100.756) (width 1.7) (layer F.Cu) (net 2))
 (segment (start 149.336 103.796) (end 149.54 104) (width 1.7) (layer F.Cu) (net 2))
 (segment (start 149.58 103.96) (end 149.54 104) (width 1.7) (layer F.Cu) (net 2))
 (segment (start 149.58 97.976) (end 149.58 103.96) (width 1.7) (layer F.Cu) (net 2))
 (segment (start 144.5 97.976) (end 144.5 100.974) (width 1.7) (layer F.Cu) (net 3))
 (segment (start 144.55 103.91) (end 144.46 104) (width 1.7) (layer F.Cu) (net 3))
 (segment (start 144.5 103.96) (end 144.46 104) (width 1.7) (layer F.Cu) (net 3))
 (segment (start 144.5 97.976) (end 144.5 103.96) (width 1.7) (layer F.Cu) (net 3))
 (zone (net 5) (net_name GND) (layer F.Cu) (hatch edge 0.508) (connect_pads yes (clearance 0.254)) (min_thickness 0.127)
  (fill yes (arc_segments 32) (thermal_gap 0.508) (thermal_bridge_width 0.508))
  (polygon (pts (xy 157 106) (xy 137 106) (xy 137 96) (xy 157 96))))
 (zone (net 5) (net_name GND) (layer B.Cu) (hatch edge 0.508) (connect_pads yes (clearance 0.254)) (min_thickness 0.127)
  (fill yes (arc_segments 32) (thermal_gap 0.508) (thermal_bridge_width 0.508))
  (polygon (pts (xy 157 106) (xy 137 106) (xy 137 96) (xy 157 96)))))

